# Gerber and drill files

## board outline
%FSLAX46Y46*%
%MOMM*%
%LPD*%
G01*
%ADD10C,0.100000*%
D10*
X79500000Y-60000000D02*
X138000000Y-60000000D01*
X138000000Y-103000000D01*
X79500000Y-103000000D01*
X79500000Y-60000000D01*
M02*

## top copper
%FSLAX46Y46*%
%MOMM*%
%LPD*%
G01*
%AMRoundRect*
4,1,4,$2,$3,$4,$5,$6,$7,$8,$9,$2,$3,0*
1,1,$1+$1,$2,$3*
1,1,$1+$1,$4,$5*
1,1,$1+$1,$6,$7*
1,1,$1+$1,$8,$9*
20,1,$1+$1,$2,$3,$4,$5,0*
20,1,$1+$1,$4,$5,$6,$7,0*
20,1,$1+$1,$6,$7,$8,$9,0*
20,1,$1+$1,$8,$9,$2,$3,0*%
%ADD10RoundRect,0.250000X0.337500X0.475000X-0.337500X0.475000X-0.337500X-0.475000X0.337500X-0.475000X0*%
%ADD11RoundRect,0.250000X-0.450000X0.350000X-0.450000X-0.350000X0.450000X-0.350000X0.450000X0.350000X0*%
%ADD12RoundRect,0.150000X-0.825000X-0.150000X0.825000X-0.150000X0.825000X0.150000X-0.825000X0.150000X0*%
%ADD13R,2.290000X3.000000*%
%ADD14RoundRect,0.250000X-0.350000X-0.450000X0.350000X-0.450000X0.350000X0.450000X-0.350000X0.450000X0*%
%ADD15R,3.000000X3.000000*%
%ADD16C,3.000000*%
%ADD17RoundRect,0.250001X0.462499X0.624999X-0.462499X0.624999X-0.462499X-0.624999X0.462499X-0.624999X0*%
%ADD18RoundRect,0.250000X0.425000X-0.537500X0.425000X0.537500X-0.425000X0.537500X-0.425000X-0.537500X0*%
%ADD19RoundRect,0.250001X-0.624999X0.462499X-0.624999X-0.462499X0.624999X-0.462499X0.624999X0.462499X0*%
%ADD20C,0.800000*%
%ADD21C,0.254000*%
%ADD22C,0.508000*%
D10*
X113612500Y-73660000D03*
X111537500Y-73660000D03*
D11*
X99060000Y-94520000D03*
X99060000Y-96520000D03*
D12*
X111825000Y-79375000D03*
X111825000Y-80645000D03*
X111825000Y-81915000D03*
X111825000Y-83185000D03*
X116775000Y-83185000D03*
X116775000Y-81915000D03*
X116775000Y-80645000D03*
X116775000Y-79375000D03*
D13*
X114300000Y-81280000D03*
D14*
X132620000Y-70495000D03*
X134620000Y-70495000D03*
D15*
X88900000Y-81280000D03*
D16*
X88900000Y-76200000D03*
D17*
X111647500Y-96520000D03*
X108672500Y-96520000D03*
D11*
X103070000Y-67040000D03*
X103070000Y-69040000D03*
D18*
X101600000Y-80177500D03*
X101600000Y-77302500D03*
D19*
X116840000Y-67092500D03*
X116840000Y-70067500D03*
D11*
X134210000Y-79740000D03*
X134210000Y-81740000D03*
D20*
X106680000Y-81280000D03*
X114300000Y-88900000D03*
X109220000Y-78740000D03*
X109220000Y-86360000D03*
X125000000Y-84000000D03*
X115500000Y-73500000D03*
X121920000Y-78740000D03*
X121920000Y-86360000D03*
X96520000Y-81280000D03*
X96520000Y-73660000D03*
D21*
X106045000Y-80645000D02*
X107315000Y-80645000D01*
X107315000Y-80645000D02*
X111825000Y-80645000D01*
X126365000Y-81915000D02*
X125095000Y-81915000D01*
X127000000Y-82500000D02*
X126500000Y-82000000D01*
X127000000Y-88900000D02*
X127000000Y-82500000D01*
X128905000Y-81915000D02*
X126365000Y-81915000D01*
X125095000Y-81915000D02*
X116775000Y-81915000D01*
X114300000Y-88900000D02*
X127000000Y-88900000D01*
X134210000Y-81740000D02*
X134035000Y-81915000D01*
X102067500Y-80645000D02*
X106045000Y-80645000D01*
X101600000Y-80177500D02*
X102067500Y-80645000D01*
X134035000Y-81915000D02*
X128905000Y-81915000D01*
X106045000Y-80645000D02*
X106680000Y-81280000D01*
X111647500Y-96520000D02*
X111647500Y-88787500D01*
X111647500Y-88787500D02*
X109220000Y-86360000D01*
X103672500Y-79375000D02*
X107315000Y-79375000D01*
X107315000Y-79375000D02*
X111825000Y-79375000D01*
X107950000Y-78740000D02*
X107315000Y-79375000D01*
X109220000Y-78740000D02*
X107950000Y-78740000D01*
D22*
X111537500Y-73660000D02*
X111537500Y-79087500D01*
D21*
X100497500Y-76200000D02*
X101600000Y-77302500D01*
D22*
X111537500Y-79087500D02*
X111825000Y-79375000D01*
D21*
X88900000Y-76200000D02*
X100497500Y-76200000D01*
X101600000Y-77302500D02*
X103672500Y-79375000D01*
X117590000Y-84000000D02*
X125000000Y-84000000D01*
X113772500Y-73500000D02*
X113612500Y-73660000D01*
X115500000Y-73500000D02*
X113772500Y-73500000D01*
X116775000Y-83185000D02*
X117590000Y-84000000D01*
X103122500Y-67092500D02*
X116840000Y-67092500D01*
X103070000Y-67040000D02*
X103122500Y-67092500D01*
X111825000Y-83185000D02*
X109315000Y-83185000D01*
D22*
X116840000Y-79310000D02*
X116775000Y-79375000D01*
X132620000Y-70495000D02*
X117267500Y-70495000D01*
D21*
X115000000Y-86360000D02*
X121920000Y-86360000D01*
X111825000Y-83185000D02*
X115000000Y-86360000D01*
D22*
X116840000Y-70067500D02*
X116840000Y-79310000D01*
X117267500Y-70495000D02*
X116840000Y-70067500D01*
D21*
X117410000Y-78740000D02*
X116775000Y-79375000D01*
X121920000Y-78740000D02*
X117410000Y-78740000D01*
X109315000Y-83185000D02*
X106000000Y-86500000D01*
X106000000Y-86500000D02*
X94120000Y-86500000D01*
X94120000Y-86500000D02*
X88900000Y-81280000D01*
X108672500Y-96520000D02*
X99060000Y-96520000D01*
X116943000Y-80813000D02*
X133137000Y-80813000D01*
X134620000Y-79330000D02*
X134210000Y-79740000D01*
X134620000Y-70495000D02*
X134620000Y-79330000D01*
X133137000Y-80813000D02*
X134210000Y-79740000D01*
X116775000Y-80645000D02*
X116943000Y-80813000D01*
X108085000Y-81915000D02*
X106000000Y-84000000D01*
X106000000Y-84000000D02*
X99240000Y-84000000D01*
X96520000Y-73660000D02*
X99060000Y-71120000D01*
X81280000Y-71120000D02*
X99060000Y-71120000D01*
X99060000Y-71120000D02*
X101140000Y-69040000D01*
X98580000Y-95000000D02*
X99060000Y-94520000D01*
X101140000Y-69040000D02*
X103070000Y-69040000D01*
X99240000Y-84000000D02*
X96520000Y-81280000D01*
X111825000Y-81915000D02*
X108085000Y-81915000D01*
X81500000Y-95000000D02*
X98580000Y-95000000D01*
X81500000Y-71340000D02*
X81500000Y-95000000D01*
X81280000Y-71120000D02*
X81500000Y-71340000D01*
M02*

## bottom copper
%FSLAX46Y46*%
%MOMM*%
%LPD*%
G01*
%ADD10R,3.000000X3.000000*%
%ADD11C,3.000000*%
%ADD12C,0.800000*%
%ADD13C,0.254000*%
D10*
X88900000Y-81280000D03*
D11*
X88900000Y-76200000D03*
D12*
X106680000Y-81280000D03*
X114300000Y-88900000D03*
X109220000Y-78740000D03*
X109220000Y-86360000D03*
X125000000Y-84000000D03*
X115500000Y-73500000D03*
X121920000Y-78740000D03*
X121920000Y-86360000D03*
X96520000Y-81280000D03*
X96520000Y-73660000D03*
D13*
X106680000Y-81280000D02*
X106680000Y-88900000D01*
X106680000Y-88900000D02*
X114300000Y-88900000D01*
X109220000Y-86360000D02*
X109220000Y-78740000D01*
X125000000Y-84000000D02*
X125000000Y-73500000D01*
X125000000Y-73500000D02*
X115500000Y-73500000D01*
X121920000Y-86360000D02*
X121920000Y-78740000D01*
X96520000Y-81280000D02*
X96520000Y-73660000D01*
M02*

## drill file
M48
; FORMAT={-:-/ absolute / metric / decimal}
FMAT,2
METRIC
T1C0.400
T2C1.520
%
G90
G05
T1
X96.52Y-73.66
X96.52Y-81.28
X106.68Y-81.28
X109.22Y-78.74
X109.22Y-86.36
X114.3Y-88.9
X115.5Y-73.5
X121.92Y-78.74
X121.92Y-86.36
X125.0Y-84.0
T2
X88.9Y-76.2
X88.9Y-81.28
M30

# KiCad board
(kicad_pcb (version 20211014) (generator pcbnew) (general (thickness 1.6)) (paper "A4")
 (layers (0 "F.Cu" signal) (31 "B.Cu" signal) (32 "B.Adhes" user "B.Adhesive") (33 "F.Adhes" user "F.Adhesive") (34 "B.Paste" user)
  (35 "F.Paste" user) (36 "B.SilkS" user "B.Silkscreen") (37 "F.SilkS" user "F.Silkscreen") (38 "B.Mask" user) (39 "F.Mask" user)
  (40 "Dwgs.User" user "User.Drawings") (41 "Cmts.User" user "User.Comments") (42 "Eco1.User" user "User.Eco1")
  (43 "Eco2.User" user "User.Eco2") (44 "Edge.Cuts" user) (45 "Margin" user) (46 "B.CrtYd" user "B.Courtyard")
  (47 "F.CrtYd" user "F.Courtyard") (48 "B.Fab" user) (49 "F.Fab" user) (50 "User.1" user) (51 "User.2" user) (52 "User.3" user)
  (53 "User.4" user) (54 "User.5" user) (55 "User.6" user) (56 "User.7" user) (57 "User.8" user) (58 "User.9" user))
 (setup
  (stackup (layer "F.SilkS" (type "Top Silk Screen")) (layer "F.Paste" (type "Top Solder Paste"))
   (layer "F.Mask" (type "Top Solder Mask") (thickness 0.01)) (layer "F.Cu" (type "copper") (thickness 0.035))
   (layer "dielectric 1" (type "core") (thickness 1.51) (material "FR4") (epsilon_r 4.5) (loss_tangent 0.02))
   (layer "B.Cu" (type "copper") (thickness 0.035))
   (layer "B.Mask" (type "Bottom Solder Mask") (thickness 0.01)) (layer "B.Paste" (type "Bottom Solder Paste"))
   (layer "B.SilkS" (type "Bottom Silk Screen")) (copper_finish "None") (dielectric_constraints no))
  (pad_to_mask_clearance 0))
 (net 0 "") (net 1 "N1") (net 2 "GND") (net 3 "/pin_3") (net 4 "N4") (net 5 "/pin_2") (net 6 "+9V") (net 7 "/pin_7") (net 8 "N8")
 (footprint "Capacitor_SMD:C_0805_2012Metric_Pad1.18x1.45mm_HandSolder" (layer "F.Cu") (at 112.575 73.66 180)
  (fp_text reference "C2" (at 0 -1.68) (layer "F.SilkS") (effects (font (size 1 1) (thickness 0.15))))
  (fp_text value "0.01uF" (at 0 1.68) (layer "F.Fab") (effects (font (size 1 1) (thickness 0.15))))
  (pad "1" smd roundrect (at -1.0375 0 180) (size 1.175 1.45) (layers "F.Cu" "F.Paste" "F.Mask") (roundrect_rratio 0.212766) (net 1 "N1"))
  (pad "2" smd roundrect (at 1.0375 0 180) (size 1.175 1.45) (layers "F.Cu" "F.Paste" "F.Mask") (roundrect_rratio 0.212766) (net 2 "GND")))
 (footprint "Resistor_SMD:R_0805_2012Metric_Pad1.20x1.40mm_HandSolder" (layer "F.Cu") (at 99.06 95.52 -90)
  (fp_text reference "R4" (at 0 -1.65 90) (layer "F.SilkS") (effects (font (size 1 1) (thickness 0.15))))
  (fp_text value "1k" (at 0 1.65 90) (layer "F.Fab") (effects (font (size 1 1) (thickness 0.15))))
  (pad "1" smd roundrect (at -1 0 270) (size 1.2 1.4) (layers "F.Cu" "F.Paste" "F.Mask") (roundrect_rratio 0.208333) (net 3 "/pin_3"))
  (pad "2" smd roundrect (at 1 0 270) (size 1.2 1.4) (layers "F.Cu" "F.Paste" "F.Mask") (roundrect_rratio 0.208333) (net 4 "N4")))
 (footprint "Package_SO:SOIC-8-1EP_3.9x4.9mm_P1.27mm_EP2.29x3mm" (layer "F.Cu") (at 114.3 81.28)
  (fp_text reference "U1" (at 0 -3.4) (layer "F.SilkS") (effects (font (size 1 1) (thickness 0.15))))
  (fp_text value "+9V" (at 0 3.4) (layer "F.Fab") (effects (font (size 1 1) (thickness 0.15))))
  (pad "" smd roundrect (at 0.57 0.75) (size 0.92 1.21) (layers "F.Paste") (roundrect_rratio 0.25))
  (pad "" smd roundrect (at 0.57 -0.75) (size 0.92 1.21) (layers "F.Paste") (roundrect_rratio 0.25))
  (pad "" smd roundrect (at -0.57 -0.75) (size 0.92 1.21) (layers "F.Paste") (roundrect_rratio 0.25))
  (pad "" smd roundrect (at -0.57 0.75) (size 0.92 1.21) (layers "F.Paste") (roundrect_rratio 0.25))
  (pad "1" smd roundrect (at -2.475 -1.905) (size 1.95 0.6) (layers "F.Cu" "F.Paste" "F.Mask") (roundrect_rratio 0.25) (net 2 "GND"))
  (pad "2" smd roundrect (at -2.475 -0.635) (size 1.95 0.6) (layers "F.Cu" "F.Paste" "F.Mask") (roundrect_rratio 0.25) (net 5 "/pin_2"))
  (pad "3" smd roundrect (at -2.475 0.635) (size 1.95 0.6) (layers "F.Cu" "F.Paste" "F.Mask") (roundrect_rratio 0.25) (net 3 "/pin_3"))
  (pad "4" smd roundrect (at -2.475 1.905) (size 1.95 0.6) (layers "F.Cu" "F.Paste" "F.Mask") (roundrect_rratio 0.25) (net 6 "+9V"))
  (pad "5" smd roundrect (at 2.475 1.905) (size 1.95 0.6) (layers "F.Cu" "F.Paste" "F.Mask") (roundrect_rratio 0.25) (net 1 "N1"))
  (pad "6" smd roundrect (at 2.475 0.635) (size 1.95 0.6) (layers "F.Cu" "F.Paste" "F.Mask") (roundrect_rratio 0.25) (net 5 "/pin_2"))
  (pad "7" smd roundrect (at 2.475 -0.635) (size 1.95 0.6) (layers "F.Cu" "F.Paste" "F.Mask") (roundrect_rratio 0.25) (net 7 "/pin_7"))
  (pad "8" smd roundrect (at 2.475 -1.905) (size 1.95 0.6) (layers "F.Cu" "F.Paste" "F.Mask") (roundrect_rratio 0.25) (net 6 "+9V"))
  (pad "9" smd rect (at 0 0) (size 2.29 3) (layers "F.Cu" "F.Mask")))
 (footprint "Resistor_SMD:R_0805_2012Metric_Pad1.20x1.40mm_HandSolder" (layer "F.Cu") (at 133.62 70.495)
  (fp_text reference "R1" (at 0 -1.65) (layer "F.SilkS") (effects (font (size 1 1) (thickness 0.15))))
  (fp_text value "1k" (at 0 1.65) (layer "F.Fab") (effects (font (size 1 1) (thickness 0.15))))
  (pad "1" smd roundrect (at -1 0) (size 1.2 1.4) (layers "F.Cu" "F.Paste" "F.Mask") (roundrect_rratio 0.208333) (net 6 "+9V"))
  (pad "2" smd roundrect (at 1 0) (size 1.2 1.4) (layers "F.Cu" "F.Paste" "F.Mask") (roundrect_rratio 0.208333) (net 7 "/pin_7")))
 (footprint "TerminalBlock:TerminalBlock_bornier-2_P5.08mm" (layer "F.Cu") (at 88.9 81.28 90)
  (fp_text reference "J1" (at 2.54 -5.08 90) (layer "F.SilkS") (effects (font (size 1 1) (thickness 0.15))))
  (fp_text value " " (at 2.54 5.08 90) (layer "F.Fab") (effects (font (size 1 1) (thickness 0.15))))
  (pad "1" thru_hole rect (at 0 0 90) (size 3 3) (drill 1.52) (layers *.Cu *.Mask) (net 6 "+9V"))
  (pad "2" thru_hole circle (at 5.08 0 90) (size 3 3) (drill 1.52) (layers *.Cu *.Mask) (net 2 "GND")))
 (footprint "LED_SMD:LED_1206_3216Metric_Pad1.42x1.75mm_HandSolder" (layer "F.Cu") (at 110.16 96.52 180)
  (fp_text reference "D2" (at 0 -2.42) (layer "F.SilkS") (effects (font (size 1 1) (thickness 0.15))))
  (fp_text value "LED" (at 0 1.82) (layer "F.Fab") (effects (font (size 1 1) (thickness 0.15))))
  (pad "1" smd roundrect (at -1.4875 0 180) (size 1.425 1.75) (layers "F.Cu" "F.Paste" "F.Mask") (roundrect_rratio 0.175439) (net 2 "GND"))
  (pad "2" smd roundrect (at 1.4875 0 180) (size 1.425 1.75) (layers "F.Cu" "F.Paste" "F.Mask") (roundrect_rratio 0.175439) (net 4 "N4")))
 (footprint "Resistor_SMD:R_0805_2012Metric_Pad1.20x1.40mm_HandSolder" (layer "F.Cu") (at 103.07 68.04 -90)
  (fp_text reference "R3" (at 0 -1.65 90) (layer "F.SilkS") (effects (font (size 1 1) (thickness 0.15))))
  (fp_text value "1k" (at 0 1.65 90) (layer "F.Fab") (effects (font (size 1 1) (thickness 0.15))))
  (pad "1" smd roundrect (at -1 0 270) (size 1.2 1.4) (layers "F.Cu" "F.Paste" "F.Mask") (roundrect_rratio 0.208333) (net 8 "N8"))
  (pad "2" smd roundrect (at 1 0 270) (size 1.2 1.4) (layers "F.Cu" "F.Paste" "F.Mask") (roundrect_rratio 0.208333) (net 3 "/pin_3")))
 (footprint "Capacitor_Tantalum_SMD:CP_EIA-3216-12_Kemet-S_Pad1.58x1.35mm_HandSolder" (layer "F.Cu") (at 101.6 78.74 90)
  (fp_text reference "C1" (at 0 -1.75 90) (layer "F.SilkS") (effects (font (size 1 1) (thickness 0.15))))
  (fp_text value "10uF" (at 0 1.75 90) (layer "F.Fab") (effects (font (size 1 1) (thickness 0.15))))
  (pad "1" smd roundrect (at -1.4375 0 90) (size 1.575 1.35) (layers "F.Cu" "F.Paste" "F.Mask") (roundrect_rratio 0.185185) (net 5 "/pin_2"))
  (pad "2" smd roundrect (at 1.4375 0 90) (size 1.575 1.35) (layers "F.Cu" "F.Paste" "F.Mask") (roundrect_rratio 0.185185) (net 2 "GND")))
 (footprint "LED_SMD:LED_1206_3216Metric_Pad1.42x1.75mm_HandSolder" (layer "F.Cu") (at 116.84 68.58 -90)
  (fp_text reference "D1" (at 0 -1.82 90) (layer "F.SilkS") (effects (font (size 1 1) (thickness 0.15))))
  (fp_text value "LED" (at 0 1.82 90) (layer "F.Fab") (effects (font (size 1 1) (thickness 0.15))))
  (pad "1" smd roundrect (at -1.4875 0 270) (size 1.425 1.75) (layers "F.Cu" "F.Paste" "F.Mask") (roundrect_rratio 0.175439) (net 8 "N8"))
  (pad "2" smd roundrect (at 1.4875 0 270) (size 1.425 1.75) (layers "F.Cu" "F.Paste" "F.Mask") (roundrect_rratio 0.175439) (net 6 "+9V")))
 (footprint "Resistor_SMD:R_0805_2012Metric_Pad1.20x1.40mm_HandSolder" (layer "F.Cu") (at 134.21 80.74 -90)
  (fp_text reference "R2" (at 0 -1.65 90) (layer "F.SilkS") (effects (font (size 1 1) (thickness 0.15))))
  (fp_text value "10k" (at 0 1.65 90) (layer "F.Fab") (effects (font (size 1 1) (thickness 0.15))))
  (pad "1" smd roundrect (at -1 0 270) (size 1.2 1.4) (layers "F.Cu" "F.Paste" "F.Mask") (roundrect_rratio 0.208333) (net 7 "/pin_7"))
  (pad "2" smd roundrect (at 1 0 270) (size 1.2 1.4) (layers "F.Cu" "F.Paste" "F.Mask") (roundrect_rratio 0.208333) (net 5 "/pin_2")))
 (gr_rect (start 79.5 60) (end 138 103) (layer "Edge.Cuts") (width 0.1) (fill none))
 (segment (start 106.045 80.645) (end 107.315 80.645) (width 0.254) (layer "F.Cu") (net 5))
 (segment (start 107.315 80.645) (end 111.825 80.645) (width 0.254) (layer "F.Cu") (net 5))
 (segment (start 126.365 81.915) (end 125.095 81.915) (width 0.254) (layer "F.Cu") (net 5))
 (segment (start 127 82.5) (end 126.5 82) (width 0.254) (layer "F.Cu") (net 5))
 (segment (start 127 88.9) (end 127 82.5) (width 0.254) (layer "F.Cu") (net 5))
 (segment (start 128.905 81.915) (end 126.365 81.915) (width 0.254) (layer "F.Cu") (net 5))
 (segment (start 125.095 81.915) (end 116.775 81.915) (width 0.254) (layer "F.Cu") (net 5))
 (segment (start 114.3 88.9) (end 127 88.9) (width 0.254) (layer "F.Cu") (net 5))
 (segment (start 134.21 81.74) (end 134.035 81.915) (width 0.254) (layer "F.Cu") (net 5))
 (segment (start 102.0675 80.645) (end 106.045 80.645) (width 0.254) (layer "F.Cu") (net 5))
 (segment (start 101.6 80.1775) (end 102.0675 80.645) (width 0.254) (layer "F.Cu") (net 5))
 (segment (start 134.035 81.915) (end 128.905 81.915) (width 0.254) (layer "F.Cu") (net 5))
 (segment (start 106.045 80.645) (end 106.68 81.28) (width 0.254) (layer "F.Cu") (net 5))
 (via (at 106.68 81.28) (size 0.8) (drill 0.4) (layers "F.Cu" "B.Cu") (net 5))
 (via (at 114.3 88.9) (size 0.8) (drill 0.4) (layers "F.Cu" "B.Cu") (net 5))
 (segment (start 106.68 81.28) (end 106.68 88.9) (width 0.254) (layer "B.Cu") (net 5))
 (segment (start 106.68 88.9) (end 114.3 88.9) (width 0.254) (layer "B.Cu") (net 5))
 (segment (start 111.6475 96.52) (end 111.6475 88.7875) (width 0.254) (layer "F.Cu") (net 2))
 (segment (start 111.6475 88.7875) (end 109.22 86.36) (width 0.254) (layer "F.Cu") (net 2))
 (segment (start 103.6725 79.375) (end 107.315 79.375) (width 0.254) (layer "F.Cu") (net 2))
 (segment (start 107.315 79.375) (end 111.825 79.375) (width 0.254) (layer "F.Cu") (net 2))
 (segment (start 107.95 78.74) (end 107.315 79.375) (width 0.254) (layer "F.Cu") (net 2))
 (segment (start 109.22 78.74) (end 107.95 78.74) (width 0.254) (layer "F.Cu") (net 2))
 (segment (start 111.5375 73.66) (end 111.5375 79.0875) (width 0.508) (layer "F.Cu") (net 2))
 (segment (start 100.4975 76.2) (end 101.6 77.3025) (width 0.254) (layer "F.Cu") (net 2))
 (segment (start 111.5375 79.0875) (end 111.825 79.375) (width 0.508) (layer "F.Cu") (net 2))
 (segment (start 88.9 76.2) (end 100.4975 76.2) (width 0.254) (layer "F.Cu") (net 2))
 (segment (start 101.6 77.3025) (end 103.6725 79.375) (width 0.254) (layer "F.Cu") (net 2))
 (via (at 109.22 78.74) (size 0.8) (drill 0.4) (layers "F.Cu" "B.Cu") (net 2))
 (via (at 109.22 86.36) (size 0.8) (drill 0.4) (layers "F.Cu" "B.Cu") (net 2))
 (segment (start 109.22 86.36) (end 109.22 78.74) (width 0.254) (layer "B.Cu") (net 2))
 (segment (start 117.59 84) (end 125 84) (width 0.254) (layer "F.Cu") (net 1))
 (segment (start 113.7725 73.5) (end 113.6125 73.66) (width 0.254) (layer "F.Cu") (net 1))
 (segment (start 115.5 73.5) (end 113.7725 73.5) (width 0.254) (layer "F.Cu") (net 1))
 (segment (start 116.775 83.185) (end 117.59 84) (width 0.254) (layer "F.Cu") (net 1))
 (via (at 125 84) (size 0.8) (drill 0.4) (layers "F.Cu" "B.Cu") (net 1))
 (via (at 115.5 73.5) (size 0.8) (drill 0.4) (layers "F.Cu" "B.Cu") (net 1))
 (segment (start 125 84) (end 125 73.5) (width 0.254) (layer "B.Cu") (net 1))
 (segment (start 125 73.5) (end 115.5 73.5) (width 0.254) (layer "B.Cu") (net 1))
 (segment (start 103.1225 67.0925) (end 116.84 67.0925) (width 0.254) (layer "F.Cu") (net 8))
 (segment (start 103.07 67.04) (end 103.1225 67.0925) (width 0.254) (layer "F.Cu") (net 8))
 (segment (start 111.825 83.185) (end 109.315 83.185) (width 0.254) (layer "F.Cu") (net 6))
 (segment (start 116.84 79.31) (end 116.775 79.375) (width 0.508) (layer "F.Cu") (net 6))
 (segment (start 132.62 70.495) (end 117.2675 70.495) (width 0.508) (layer "F.Cu") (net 6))
 (segment (start 115 86.36) (end 121.92 86.36) (width 0.254) (layer "F.Cu") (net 6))
 (segment (start 111.825 83.185) (end 115 86.36) (width 0.254) (layer "F.Cu") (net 6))
 (segment (start 116.84 70.0675) (end 116.84 79.31) (width 0.508) (layer "F.Cu") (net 6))
 (segment (start 117.2675 70.495) (end 116.84 70.0675) (width 0.508) (layer "F.Cu") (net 6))
 (segment (start 117.41 78.74) (end 116.775 79.375) (width 0.254) (layer "F.Cu") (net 6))
 (segment (start 121.92 78.74) (end 117.41 78.74) (width 0.254) (layer "F.Cu") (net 6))
 (segment (start 109.315 83.185) (end 106 86.5) (width 0.254) (layer "F.Cu") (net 6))
 (segment (start 106 86.5) (end 94.12 86.5) (width 0.254) (layer "F.Cu") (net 6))
 (segment (start 94.12 86.5) (end 88.9 81.28) (width 0.254) (layer "F.Cu") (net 6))
 (via (at 121.92 78.74) (size 0.8) (drill 0.4) (layers "F.Cu" "B.Cu") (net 6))
 (via (at 121.92 86.36) (size 0.8) (drill 0.4) (layers "F.Cu" "B.Cu") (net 6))
 (segment (start 121.92 86.36) (end 121.92 78.74) (width 0.254) (layer "B.Cu") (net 6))
 (segment (start 108.6725 96.52) (end 99.06 96.52) (width 0.254) (layer "F.Cu") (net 4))
 (segment (start 116.943 80.813) (end 133.137 80.813) (width 0.254) (layer "F.Cu") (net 7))
 (segment (start 134.62 79.33) (end 134.21 79.74) (width 0.254) (layer "F.Cu") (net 7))
 (segment (start 134.62 70.495) (end 134.62 79.33) (width 0.254) (layer "F.Cu") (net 7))
 (segment (start 133.137 80.813) (end 134.21 79.74) (width 0.254) (layer "F.Cu") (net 7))
 (segment (start 116.775 80.645) (end 116.943 80.813) (width 0.254) (layer "F.Cu") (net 7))
 (segment (start 108.085 81.915) (end 106 84) (width 0.254) (layer "F.Cu") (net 3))
 (segment (start 106 84) (end 99.24 84) (width 0.254) (layer "F.Cu") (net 3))
 (segment (start 96.52 73.66) (end 99.06 71.12) (width 0.254) (layer "F.Cu") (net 3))
 (segment (start 81.28 71.12) (end 99.06 71.12) (width 0.254) (layer "F.Cu") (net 3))
 (segment (start 99.06 71.12) (end 101.14 69.04) (width 0.254) (layer "F.Cu") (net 3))
 (segment (start 98.58 95) (end 99.06 94.52) (width 0.254) (layer "F.Cu") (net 3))
 (segment (start 101.14 69.04) (end 103.07 69.04) (width 0.254) (layer "F.Cu") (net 3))
 (segment (start 99.24 84) (end 96.52 81.28) (width 0.254) (layer "F.Cu") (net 3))
 (segment (start 111.825 81.915) (end 108.085 81.915) (width 0.254) (layer "F.Cu") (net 3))
 (segment (start 81.5 95) (end 98.58 95) (width 0.254) (layer "F.Cu") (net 3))
 (segment (start 81.5 71.34) (end 81.5 95) (width 0.254) (layer "F.Cu") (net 3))
 (segment (start 81.28 71.12) (end 81.5 71.34) (width 0.254) (layer "F.Cu") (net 3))
 (via (at 96.52 81.28) (size 0.8) (drill 0.4) (layers "F.Cu" "B.Cu") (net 3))
 (via (at 96.52 73.66) (size 0.8) (drill 0.4) (layers "F.Cu" "B.Cu") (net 3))
 (segment (start 96.52 81.28) (end 96.52 73.66) (width 0.254) (layer "B.Cu") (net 3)))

